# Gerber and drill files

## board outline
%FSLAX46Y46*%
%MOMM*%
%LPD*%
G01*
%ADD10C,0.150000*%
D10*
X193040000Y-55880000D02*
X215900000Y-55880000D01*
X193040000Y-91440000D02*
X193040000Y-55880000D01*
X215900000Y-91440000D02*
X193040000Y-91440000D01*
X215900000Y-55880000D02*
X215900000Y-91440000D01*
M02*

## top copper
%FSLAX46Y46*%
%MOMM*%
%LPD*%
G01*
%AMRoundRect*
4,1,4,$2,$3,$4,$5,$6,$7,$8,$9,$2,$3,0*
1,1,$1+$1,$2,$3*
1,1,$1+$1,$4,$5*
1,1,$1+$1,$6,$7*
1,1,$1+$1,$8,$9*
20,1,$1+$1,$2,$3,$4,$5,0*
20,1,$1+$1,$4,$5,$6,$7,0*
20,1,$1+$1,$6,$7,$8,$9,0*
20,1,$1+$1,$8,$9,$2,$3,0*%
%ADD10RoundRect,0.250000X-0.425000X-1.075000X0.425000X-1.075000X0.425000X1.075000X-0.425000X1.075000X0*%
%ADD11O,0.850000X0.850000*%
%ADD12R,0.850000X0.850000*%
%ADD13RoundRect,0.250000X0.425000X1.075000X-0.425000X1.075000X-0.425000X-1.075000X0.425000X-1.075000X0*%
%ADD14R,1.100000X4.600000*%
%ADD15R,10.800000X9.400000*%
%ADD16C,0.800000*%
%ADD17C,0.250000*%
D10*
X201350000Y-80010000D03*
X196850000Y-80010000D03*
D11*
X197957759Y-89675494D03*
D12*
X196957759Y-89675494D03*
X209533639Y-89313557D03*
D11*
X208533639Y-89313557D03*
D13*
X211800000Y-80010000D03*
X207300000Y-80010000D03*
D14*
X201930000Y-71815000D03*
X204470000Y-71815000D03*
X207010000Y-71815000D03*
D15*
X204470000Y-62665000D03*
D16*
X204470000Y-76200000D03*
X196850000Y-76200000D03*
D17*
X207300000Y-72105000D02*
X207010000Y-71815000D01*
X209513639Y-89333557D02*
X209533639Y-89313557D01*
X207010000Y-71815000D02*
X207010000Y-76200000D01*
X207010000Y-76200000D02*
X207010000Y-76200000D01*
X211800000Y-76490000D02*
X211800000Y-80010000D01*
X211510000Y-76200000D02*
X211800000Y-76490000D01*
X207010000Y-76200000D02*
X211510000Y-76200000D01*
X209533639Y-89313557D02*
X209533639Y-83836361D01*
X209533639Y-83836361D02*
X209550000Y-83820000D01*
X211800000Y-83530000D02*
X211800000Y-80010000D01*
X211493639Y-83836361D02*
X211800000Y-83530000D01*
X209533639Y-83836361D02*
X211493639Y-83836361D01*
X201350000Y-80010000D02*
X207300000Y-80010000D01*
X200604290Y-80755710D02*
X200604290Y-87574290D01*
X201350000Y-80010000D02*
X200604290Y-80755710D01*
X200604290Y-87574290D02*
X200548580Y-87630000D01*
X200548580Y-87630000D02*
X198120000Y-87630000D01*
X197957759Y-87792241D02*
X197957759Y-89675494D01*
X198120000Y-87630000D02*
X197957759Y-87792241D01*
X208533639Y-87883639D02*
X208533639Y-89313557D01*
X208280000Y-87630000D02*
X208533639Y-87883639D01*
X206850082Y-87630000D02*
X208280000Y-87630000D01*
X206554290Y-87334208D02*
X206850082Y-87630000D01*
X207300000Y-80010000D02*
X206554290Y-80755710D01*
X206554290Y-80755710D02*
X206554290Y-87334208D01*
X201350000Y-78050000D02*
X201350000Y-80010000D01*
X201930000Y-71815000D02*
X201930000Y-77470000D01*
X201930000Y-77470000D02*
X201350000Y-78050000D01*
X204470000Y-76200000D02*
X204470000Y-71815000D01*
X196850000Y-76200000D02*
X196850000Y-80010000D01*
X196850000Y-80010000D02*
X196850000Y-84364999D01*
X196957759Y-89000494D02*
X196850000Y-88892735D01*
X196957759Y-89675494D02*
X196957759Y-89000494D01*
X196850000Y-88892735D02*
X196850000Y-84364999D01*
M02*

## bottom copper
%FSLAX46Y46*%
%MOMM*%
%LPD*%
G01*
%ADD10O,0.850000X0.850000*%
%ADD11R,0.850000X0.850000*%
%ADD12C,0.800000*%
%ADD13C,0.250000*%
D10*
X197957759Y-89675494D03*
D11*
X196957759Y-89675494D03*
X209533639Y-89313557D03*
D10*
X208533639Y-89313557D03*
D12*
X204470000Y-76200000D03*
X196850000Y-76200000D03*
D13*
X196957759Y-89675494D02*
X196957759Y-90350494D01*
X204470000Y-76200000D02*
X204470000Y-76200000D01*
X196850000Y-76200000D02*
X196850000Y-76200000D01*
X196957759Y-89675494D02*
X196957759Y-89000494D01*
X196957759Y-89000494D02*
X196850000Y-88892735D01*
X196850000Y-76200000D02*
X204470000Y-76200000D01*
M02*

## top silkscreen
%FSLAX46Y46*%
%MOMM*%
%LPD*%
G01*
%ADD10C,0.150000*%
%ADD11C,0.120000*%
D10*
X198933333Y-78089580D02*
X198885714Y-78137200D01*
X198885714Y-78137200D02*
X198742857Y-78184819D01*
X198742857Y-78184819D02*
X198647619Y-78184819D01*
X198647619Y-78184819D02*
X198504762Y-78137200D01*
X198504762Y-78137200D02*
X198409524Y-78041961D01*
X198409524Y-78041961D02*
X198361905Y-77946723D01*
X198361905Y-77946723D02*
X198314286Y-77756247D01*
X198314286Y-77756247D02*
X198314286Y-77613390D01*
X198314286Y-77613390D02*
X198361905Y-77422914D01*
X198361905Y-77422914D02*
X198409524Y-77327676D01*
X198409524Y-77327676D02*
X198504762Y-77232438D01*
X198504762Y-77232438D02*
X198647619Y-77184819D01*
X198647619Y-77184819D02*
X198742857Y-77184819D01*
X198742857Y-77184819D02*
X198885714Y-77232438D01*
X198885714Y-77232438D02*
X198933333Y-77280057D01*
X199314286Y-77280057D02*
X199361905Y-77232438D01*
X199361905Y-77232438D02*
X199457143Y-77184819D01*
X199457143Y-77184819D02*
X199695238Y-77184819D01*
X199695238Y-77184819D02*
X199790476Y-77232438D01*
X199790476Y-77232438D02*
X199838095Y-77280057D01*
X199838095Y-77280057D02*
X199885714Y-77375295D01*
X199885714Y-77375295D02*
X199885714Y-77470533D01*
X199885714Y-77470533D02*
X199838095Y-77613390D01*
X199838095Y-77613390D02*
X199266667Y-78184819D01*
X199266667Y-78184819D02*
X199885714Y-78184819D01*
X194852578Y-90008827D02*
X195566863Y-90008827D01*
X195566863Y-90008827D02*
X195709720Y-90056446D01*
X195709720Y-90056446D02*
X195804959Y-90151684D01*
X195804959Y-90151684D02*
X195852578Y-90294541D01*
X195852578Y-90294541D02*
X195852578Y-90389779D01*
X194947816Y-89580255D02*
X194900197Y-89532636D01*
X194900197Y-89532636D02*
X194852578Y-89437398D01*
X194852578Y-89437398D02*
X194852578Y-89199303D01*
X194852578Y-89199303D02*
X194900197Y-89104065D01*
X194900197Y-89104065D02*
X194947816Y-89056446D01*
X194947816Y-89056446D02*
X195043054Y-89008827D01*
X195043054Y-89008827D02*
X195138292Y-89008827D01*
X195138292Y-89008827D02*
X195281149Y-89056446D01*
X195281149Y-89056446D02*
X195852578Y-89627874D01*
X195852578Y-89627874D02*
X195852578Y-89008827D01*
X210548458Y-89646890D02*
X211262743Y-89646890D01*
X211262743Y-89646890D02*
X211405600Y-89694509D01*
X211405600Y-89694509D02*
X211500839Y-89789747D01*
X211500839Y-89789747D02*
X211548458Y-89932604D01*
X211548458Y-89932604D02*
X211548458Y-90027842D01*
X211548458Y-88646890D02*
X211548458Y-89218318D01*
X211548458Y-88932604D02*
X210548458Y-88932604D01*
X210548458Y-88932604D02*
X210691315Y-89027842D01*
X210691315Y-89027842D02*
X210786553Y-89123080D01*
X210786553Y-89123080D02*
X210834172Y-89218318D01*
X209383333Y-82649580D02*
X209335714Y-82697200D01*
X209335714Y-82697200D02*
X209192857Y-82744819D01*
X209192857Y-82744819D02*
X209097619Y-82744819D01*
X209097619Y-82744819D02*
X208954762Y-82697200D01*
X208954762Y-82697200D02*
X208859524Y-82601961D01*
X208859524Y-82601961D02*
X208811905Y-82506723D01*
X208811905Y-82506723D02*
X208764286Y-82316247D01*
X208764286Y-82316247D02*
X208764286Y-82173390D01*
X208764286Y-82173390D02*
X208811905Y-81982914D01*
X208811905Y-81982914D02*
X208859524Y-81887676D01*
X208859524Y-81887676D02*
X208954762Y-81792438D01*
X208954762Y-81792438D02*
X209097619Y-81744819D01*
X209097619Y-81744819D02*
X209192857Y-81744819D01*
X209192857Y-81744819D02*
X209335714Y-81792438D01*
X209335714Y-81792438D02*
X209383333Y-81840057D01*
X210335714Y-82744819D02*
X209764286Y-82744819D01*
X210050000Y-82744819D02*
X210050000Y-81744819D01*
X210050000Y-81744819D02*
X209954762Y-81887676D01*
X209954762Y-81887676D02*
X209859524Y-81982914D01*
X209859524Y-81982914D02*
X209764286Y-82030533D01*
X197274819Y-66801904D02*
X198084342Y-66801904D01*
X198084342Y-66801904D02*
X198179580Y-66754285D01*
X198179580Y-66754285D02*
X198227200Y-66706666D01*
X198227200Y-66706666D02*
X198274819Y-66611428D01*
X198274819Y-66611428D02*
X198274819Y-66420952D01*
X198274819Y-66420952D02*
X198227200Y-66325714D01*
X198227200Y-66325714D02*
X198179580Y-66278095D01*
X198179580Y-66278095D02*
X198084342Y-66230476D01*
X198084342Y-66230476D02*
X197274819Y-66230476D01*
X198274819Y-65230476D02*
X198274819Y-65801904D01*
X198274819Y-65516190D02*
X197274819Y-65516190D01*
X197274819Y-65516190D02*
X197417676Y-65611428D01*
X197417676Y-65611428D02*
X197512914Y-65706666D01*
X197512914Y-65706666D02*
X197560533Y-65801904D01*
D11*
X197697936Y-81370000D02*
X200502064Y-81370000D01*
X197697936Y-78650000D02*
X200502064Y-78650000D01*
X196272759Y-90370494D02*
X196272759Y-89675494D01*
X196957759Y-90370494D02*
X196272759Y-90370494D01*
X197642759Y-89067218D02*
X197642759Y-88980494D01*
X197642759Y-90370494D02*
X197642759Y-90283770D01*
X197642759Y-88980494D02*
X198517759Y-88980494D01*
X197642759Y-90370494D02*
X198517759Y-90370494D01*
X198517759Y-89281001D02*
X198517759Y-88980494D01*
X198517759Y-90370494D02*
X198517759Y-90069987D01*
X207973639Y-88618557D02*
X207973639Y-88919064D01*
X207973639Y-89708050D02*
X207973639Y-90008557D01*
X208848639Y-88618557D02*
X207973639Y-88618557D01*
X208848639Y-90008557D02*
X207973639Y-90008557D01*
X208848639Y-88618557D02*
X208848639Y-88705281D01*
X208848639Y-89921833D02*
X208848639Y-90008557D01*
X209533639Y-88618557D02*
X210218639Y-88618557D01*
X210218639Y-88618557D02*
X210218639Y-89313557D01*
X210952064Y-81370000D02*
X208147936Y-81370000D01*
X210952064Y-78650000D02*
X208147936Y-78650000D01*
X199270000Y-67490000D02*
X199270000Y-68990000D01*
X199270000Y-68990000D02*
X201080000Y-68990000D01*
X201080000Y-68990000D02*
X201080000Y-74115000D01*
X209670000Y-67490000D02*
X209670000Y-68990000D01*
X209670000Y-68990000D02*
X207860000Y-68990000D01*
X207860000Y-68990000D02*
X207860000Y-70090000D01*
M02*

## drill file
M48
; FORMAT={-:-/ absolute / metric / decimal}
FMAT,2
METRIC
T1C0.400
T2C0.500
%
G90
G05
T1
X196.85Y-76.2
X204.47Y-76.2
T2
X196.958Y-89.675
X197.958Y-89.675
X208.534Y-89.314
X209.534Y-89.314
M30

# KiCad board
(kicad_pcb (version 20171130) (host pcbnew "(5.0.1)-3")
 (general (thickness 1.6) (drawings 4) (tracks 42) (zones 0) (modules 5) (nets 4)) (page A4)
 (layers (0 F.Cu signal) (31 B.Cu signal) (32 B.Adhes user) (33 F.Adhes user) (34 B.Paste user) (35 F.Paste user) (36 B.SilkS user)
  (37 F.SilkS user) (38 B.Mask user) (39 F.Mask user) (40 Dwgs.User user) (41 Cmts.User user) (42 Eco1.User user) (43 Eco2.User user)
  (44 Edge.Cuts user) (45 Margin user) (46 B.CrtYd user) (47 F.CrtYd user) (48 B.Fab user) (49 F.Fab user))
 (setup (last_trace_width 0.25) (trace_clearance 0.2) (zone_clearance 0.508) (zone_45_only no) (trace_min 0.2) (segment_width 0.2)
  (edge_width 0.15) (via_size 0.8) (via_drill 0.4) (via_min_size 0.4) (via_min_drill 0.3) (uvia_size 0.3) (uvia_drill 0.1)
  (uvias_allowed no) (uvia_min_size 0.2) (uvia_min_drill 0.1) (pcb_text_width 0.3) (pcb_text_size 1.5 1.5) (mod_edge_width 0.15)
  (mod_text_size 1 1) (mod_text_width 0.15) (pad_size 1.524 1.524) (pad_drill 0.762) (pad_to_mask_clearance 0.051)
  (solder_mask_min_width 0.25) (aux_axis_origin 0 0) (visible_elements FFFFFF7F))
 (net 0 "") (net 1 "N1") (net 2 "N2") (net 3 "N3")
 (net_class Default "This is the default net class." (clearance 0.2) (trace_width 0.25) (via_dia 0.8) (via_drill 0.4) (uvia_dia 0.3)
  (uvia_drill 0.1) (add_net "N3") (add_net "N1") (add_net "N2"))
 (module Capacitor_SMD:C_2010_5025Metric (layer F.Cu) (at 199.1 80.01)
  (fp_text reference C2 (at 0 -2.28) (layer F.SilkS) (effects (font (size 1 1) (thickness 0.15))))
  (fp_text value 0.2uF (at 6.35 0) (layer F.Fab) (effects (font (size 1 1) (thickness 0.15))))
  (fp_line (start -1.402064 1.36) (end 1.402064 1.36) (layer F.SilkS) (width 0.12))
  (fp_line (start -1.402064 -1.36) (end 1.402064 -1.36) (layer F.SilkS) (width 0.12))
  (pad 2 smd roundrect (at 2.25 0) (size 1.35 2.65) (layers F.Cu F.Paste F.Mask) (roundrect_rratio 0.185185) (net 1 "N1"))
  (pad 1 smd roundrect (at -2.25 0) (size 1.35 2.65) (layers F.Cu F.Paste F.Mask) (roundrect_rratio 0.185185) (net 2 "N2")))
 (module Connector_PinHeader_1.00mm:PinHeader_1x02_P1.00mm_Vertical (layer F.Cu) (at 196.957759 89.675494 90)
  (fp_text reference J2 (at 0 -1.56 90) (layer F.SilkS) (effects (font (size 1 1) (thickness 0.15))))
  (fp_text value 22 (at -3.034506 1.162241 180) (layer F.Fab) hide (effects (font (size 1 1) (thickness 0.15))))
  (fp_line (start -0.695 -0.685) (end 0 -0.685) (layer F.SilkS) (width 0.12))
  (fp_line (start -0.695 0) (end -0.695 -0.685) (layer F.SilkS) (width 0.12))
  (fp_line (start 0.608276 0.685) (end 0.695 0.685) (layer F.SilkS) (width 0.12))
  (fp_line (start -0.695 0.685) (end -0.608276 0.685) (layer F.SilkS) (width 0.12))
  (fp_line (start 0.695 0.685) (end 0.695 1.56) (layer F.SilkS) (width 0.12))
  (fp_line (start -0.695 0.685) (end -0.695 1.56) (layer F.SilkS) (width 0.12))
  (fp_line (start 0.394493 1.56) (end 0.695 1.56) (layer F.SilkS) (width 0.12))
  (fp_line (start -0.695 1.56) (end -0.394493 1.56) (layer F.SilkS) (width 0.12))
  (pad 2 thru_hole oval (at 0 1 90) (size 0.85 0.85) (drill 0.5) (layers *.Cu *.Mask) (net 1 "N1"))
  (pad 1 thru_hole rect (at 0 0 90) (size 0.85 0.85) (drill 0.5) (layers *.Cu *.Mask) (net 2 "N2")))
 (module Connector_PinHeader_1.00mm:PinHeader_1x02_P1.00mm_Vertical (layer F.Cu) (at 209.533639 89.313557 270)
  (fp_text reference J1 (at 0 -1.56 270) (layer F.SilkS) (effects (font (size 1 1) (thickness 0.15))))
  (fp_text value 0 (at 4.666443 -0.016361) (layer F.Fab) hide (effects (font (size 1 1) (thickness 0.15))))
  (fp_line (start -0.695 1.56) (end -0.394493 1.56) (layer F.SilkS) (width 0.12))
  (fp_line (start 0.394493 1.56) (end 0.695 1.56) (layer F.SilkS) (width 0.12))
  (fp_line (start -0.695 0.685) (end -0.695 1.56) (layer F.SilkS) (width 0.12))
  (fp_line (start 0.695 0.685) (end 0.695 1.56) (layer F.SilkS) (width 0.12))
  (fp_line (start -0.695 0.685) (end -0.608276 0.685) (layer F.SilkS) (width 0.12))
  (fp_line (start 0.608276 0.685) (end 0.695 0.685) (layer F.SilkS) (width 0.12))
  (fp_line (start -0.695 0) (end -0.695 -0.685) (layer F.SilkS) (width 0.12))
  (fp_line (start -0.695 -0.685) (end 0 -0.685) (layer F.SilkS) (width 0.12))
  (pad 1 thru_hole rect (at 0 0 270) (size 0.85 0.85) (drill 0.5) (layers *.Cu *.Mask) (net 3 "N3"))
  (pad 2 thru_hole oval (at 0 1 270) (size 0.85 0.85) (drill 0.5) (layers *.Cu *.Mask) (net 1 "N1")))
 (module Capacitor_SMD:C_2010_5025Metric (layer F.Cu) (at 209.55 80.01 180)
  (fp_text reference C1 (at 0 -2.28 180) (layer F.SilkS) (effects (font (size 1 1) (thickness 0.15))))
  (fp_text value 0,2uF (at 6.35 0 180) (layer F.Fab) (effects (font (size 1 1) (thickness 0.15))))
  (fp_line (start -1.402064 -1.36) (end 1.402064 -1.36) (layer F.SilkS) (width 0.12))
  (fp_line (start -1.402064 1.36) (end 1.402064 1.36) (layer F.SilkS) (width 0.12))
  (pad 1 smd roundrect (at -2.25 0 180) (size 1.35 2.65) (layers F.Cu F.Paste F.Mask) (roundrect_rratio 0.185185) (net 3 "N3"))
  (pad 2 smd roundrect (at 2.25 0 180) (size 1.35 2.65) (layers F.Cu F.Paste F.Mask) (roundrect_rratio 0.185185) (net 1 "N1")))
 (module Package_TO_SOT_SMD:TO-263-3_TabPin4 (layer F.Cu) (at 204.47 66.04 90)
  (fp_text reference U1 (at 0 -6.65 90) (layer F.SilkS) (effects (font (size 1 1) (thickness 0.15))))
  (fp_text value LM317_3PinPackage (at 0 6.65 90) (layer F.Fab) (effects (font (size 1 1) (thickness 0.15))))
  (fp_line (start -1.45 -5.2) (end -2.95 -5.2) (layer F.SilkS) (width 0.12))
  (fp_line (start -2.95 -5.2) (end -2.95 -3.39) (layer F.SilkS) (width 0.12))
  (fp_line (start -2.95 -3.39) (end -8.075 -3.39) (layer F.SilkS) (width 0.12))
  (fp_line (start -1.45 5.2) (end -2.95 5.2) (layer F.SilkS) (width 0.12))
  (fp_line (start -2.95 5.2) (end -2.95 3.39) (layer F.SilkS) (width 0.12))
  (fp_line (start -2.95 3.39) (end -4.05 3.39) (layer F.SilkS) (width 0.12))
  (pad 1 smd rect (at -5.775 -2.54 90) (size 4.6 1.1) (layers F.Cu F.Paste F.Mask) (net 1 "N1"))
  (pad 2 smd rect (at -5.775 0 90) (size 4.6 1.1) (layers F.Cu F.Paste F.Mask) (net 2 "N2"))
  (pad 3 smd rect (at -5.775 2.54 90) (size 4.6 1.1) (layers F.Cu F.Paste F.Mask) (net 3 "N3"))
  (pad 4 smd rect (at 3.375 0 90) (size 9.4 10.8) (layers F.Cu F.Mask))
  (pad "" smd rect (at 5.8 2.775 90) (size 4.55 5.25) (layers F.Paste))
  (pad "" smd rect (at 0.95 -2.775 90) (size 4.55 5.25) (layers F.Paste))
  (pad "" smd rect (at 5.8 -2.775 90) (size 4.55 5.25) (layers F.Paste))
  (pad "" smd rect (at 0.95 2.775 90) (size 4.55 5.25) (layers F.Paste)))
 (gr_line (start 193.04 55.88) (end 215.9 55.88) (layer Edge.Cuts) (width 0.15))
 (gr_line (start 193.04 91.44) (end 193.04 55.88) (layer Edge.Cuts) (width 0.15))
 (gr_line (start 215.9 91.44) (end 193.04 91.44) (layer Edge.Cuts) (width 0.15))
 (gr_line (start 215.9 55.88) (end 215.9 91.44) (layer Edge.Cuts) (width 0.15))
 (segment (start 207.3 72.105) (end 207.01 71.815) (width 0.25) (layer F.Cu) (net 3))
 (segment (start 209.513639 89.333557) (end 209.533639 89.313557) (width 0.25) (layer F.Cu) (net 3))
 (segment (start 207.01 71.815) (end 207.01 76.2) (width 0.25) (layer F.Cu) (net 3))
 (segment (start 207.01 76.2) (end 207.01 76.2) (width 0.25) (layer F.Cu) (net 3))
 (segment (start 211.8 76.49) (end 211.8 80.01) (width 0.25) (layer F.Cu) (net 3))
 (segment (start 211.51 76.2) (end 211.8 76.49) (width 0.25) (layer F.Cu) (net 3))
 (segment (start 207.01 76.2) (end 211.51 76.2) (width 0.25) (layer F.Cu) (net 3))
 (segment (start 209.533639 89.313557) (end 209.533639 83.836361) (width 0.25) (layer F.Cu) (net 3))
 (segment (start 209.533639 83.836361) (end 209.55 83.82) (width 0.25) (layer F.Cu) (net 3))
 (segment (start 211.8 83.53) (end 211.8 80.01) (width 0.25) (layer F.Cu) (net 3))
 (segment (start 211.493639 83.836361) (end 211.8 83.53) (width 0.25) (layer F.Cu) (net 3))
 (segment (start 209.533639 83.836361) (end 211.493639 83.836361) (width 0.25) (layer F.Cu) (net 3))
 (segment (start 201.35 80.01) (end 207.3 80.01) (width 0.25) (layer F.Cu) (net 1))
 (segment (start 200.60429 80.75571) (end 200.60429 87.57429) (width 0.25) (layer F.Cu) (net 1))
 (segment (start 201.35 80.01) (end 200.60429 80.75571) (width 0.25) (layer F.Cu) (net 1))
 (segment (start 200.60429 87.57429) (end 200.54858 87.63) (width 0.25) (layer F.Cu) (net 1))
 (segment (start 200.54858 87.63) (end 198.12 87.63) (width 0.25) (layer F.Cu) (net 1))
 (segment (start 197.957759 87.792241) (end 197.957759 89.675494) (width 0.25) (layer F.Cu) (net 1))
 (segment (start 198.12 87.63) (end 197.957759 87.792241) (width 0.25) (layer F.Cu) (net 1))
 (segment (start 208.533639 87.883639) (end 208.533639 89.313557) (width 0.25) (layer F.Cu) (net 1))
 (segment (start 208.28 87.63) (end 208.533639 87.883639) (width 0.25) (layer F.Cu) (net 1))
 (segment (start 206.850082 87.63) (end 208.28 87.63) (width 0.25) (layer F.Cu) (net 1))
 (segment (start 206.55429 87.334208) (end 206.850082 87.63) (width 0.25) (layer F.Cu) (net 1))
 (segment (start 207.3 80.01) (end 206.55429 80.75571) (width 0.25) (layer F.Cu) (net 1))
 (segment (start 206.55429 80.75571) (end 206.55429 87.334208) (width 0.25) (layer F.Cu) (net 1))
 (segment (start 201.35 78.05) (end 201.35 80.01) (width 0.25) (layer F.Cu) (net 1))
 (segment (start 201.93 71.815) (end 201.93 77.47) (width 0.25) (layer F.Cu) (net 1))
 (segment (start 201.93 77.47) (end 201.35 78.05) (width 0.25) (layer F.Cu) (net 1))
 (segment (start 196.957759 89.675494) (end 196.957759 90.350494) (width 0.25) (layer B.Cu) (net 2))
 (segment (start 204.47 76.2) (end 204.47 76.2) (width 0.25) (layer B.Cu) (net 2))
 (via (at 204.47 76.2) (size 0.8) (drill 0.4) (layers F.Cu B.Cu) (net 2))
 (segment (start 204.47 76.2) (end 204.47 71.815) (width 0.25) (layer F.Cu) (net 2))
 (segment (start 196.85 76.2) (end 196.85 76.2) (width 0.25) (layer B.Cu) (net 2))
 (segment (start 196.957759 89.675494) (end 196.957759 89.000494) (width 0.25) (layer B.Cu) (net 2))
 (segment (start 196.957759 89.000494) (end 196.85 88.892735) (width 0.25) (layer B.Cu) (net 2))
 (segment (start 196.85 76.2) (end 204.47 76.2) (width 0.25) (layer B.Cu) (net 2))
 (via (at 196.85 76.2) (size 0.8) (drill 0.4) (layers F.Cu B.Cu) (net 2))
 (segment (start 196.85 76.2) (end 196.85 80.01) (width 0.25) (layer F.Cu) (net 2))
 (segment (start 196.85 80.01) (end 196.85 84.364999) (width 0.25) (layer F.Cu) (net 2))
 (segment (start 196.957759 89.000494) (end 196.85 88.892735) (width 0.25) (layer F.Cu) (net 2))
 (segment (start 196.957759 89.675494) (end 196.957759 89.000494) (width 0.25) (layer F.Cu) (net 2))
 (segment (start 196.85 88.892735) (end 196.85 84.364999) (width 0.25) (layer F.Cu) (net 2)))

